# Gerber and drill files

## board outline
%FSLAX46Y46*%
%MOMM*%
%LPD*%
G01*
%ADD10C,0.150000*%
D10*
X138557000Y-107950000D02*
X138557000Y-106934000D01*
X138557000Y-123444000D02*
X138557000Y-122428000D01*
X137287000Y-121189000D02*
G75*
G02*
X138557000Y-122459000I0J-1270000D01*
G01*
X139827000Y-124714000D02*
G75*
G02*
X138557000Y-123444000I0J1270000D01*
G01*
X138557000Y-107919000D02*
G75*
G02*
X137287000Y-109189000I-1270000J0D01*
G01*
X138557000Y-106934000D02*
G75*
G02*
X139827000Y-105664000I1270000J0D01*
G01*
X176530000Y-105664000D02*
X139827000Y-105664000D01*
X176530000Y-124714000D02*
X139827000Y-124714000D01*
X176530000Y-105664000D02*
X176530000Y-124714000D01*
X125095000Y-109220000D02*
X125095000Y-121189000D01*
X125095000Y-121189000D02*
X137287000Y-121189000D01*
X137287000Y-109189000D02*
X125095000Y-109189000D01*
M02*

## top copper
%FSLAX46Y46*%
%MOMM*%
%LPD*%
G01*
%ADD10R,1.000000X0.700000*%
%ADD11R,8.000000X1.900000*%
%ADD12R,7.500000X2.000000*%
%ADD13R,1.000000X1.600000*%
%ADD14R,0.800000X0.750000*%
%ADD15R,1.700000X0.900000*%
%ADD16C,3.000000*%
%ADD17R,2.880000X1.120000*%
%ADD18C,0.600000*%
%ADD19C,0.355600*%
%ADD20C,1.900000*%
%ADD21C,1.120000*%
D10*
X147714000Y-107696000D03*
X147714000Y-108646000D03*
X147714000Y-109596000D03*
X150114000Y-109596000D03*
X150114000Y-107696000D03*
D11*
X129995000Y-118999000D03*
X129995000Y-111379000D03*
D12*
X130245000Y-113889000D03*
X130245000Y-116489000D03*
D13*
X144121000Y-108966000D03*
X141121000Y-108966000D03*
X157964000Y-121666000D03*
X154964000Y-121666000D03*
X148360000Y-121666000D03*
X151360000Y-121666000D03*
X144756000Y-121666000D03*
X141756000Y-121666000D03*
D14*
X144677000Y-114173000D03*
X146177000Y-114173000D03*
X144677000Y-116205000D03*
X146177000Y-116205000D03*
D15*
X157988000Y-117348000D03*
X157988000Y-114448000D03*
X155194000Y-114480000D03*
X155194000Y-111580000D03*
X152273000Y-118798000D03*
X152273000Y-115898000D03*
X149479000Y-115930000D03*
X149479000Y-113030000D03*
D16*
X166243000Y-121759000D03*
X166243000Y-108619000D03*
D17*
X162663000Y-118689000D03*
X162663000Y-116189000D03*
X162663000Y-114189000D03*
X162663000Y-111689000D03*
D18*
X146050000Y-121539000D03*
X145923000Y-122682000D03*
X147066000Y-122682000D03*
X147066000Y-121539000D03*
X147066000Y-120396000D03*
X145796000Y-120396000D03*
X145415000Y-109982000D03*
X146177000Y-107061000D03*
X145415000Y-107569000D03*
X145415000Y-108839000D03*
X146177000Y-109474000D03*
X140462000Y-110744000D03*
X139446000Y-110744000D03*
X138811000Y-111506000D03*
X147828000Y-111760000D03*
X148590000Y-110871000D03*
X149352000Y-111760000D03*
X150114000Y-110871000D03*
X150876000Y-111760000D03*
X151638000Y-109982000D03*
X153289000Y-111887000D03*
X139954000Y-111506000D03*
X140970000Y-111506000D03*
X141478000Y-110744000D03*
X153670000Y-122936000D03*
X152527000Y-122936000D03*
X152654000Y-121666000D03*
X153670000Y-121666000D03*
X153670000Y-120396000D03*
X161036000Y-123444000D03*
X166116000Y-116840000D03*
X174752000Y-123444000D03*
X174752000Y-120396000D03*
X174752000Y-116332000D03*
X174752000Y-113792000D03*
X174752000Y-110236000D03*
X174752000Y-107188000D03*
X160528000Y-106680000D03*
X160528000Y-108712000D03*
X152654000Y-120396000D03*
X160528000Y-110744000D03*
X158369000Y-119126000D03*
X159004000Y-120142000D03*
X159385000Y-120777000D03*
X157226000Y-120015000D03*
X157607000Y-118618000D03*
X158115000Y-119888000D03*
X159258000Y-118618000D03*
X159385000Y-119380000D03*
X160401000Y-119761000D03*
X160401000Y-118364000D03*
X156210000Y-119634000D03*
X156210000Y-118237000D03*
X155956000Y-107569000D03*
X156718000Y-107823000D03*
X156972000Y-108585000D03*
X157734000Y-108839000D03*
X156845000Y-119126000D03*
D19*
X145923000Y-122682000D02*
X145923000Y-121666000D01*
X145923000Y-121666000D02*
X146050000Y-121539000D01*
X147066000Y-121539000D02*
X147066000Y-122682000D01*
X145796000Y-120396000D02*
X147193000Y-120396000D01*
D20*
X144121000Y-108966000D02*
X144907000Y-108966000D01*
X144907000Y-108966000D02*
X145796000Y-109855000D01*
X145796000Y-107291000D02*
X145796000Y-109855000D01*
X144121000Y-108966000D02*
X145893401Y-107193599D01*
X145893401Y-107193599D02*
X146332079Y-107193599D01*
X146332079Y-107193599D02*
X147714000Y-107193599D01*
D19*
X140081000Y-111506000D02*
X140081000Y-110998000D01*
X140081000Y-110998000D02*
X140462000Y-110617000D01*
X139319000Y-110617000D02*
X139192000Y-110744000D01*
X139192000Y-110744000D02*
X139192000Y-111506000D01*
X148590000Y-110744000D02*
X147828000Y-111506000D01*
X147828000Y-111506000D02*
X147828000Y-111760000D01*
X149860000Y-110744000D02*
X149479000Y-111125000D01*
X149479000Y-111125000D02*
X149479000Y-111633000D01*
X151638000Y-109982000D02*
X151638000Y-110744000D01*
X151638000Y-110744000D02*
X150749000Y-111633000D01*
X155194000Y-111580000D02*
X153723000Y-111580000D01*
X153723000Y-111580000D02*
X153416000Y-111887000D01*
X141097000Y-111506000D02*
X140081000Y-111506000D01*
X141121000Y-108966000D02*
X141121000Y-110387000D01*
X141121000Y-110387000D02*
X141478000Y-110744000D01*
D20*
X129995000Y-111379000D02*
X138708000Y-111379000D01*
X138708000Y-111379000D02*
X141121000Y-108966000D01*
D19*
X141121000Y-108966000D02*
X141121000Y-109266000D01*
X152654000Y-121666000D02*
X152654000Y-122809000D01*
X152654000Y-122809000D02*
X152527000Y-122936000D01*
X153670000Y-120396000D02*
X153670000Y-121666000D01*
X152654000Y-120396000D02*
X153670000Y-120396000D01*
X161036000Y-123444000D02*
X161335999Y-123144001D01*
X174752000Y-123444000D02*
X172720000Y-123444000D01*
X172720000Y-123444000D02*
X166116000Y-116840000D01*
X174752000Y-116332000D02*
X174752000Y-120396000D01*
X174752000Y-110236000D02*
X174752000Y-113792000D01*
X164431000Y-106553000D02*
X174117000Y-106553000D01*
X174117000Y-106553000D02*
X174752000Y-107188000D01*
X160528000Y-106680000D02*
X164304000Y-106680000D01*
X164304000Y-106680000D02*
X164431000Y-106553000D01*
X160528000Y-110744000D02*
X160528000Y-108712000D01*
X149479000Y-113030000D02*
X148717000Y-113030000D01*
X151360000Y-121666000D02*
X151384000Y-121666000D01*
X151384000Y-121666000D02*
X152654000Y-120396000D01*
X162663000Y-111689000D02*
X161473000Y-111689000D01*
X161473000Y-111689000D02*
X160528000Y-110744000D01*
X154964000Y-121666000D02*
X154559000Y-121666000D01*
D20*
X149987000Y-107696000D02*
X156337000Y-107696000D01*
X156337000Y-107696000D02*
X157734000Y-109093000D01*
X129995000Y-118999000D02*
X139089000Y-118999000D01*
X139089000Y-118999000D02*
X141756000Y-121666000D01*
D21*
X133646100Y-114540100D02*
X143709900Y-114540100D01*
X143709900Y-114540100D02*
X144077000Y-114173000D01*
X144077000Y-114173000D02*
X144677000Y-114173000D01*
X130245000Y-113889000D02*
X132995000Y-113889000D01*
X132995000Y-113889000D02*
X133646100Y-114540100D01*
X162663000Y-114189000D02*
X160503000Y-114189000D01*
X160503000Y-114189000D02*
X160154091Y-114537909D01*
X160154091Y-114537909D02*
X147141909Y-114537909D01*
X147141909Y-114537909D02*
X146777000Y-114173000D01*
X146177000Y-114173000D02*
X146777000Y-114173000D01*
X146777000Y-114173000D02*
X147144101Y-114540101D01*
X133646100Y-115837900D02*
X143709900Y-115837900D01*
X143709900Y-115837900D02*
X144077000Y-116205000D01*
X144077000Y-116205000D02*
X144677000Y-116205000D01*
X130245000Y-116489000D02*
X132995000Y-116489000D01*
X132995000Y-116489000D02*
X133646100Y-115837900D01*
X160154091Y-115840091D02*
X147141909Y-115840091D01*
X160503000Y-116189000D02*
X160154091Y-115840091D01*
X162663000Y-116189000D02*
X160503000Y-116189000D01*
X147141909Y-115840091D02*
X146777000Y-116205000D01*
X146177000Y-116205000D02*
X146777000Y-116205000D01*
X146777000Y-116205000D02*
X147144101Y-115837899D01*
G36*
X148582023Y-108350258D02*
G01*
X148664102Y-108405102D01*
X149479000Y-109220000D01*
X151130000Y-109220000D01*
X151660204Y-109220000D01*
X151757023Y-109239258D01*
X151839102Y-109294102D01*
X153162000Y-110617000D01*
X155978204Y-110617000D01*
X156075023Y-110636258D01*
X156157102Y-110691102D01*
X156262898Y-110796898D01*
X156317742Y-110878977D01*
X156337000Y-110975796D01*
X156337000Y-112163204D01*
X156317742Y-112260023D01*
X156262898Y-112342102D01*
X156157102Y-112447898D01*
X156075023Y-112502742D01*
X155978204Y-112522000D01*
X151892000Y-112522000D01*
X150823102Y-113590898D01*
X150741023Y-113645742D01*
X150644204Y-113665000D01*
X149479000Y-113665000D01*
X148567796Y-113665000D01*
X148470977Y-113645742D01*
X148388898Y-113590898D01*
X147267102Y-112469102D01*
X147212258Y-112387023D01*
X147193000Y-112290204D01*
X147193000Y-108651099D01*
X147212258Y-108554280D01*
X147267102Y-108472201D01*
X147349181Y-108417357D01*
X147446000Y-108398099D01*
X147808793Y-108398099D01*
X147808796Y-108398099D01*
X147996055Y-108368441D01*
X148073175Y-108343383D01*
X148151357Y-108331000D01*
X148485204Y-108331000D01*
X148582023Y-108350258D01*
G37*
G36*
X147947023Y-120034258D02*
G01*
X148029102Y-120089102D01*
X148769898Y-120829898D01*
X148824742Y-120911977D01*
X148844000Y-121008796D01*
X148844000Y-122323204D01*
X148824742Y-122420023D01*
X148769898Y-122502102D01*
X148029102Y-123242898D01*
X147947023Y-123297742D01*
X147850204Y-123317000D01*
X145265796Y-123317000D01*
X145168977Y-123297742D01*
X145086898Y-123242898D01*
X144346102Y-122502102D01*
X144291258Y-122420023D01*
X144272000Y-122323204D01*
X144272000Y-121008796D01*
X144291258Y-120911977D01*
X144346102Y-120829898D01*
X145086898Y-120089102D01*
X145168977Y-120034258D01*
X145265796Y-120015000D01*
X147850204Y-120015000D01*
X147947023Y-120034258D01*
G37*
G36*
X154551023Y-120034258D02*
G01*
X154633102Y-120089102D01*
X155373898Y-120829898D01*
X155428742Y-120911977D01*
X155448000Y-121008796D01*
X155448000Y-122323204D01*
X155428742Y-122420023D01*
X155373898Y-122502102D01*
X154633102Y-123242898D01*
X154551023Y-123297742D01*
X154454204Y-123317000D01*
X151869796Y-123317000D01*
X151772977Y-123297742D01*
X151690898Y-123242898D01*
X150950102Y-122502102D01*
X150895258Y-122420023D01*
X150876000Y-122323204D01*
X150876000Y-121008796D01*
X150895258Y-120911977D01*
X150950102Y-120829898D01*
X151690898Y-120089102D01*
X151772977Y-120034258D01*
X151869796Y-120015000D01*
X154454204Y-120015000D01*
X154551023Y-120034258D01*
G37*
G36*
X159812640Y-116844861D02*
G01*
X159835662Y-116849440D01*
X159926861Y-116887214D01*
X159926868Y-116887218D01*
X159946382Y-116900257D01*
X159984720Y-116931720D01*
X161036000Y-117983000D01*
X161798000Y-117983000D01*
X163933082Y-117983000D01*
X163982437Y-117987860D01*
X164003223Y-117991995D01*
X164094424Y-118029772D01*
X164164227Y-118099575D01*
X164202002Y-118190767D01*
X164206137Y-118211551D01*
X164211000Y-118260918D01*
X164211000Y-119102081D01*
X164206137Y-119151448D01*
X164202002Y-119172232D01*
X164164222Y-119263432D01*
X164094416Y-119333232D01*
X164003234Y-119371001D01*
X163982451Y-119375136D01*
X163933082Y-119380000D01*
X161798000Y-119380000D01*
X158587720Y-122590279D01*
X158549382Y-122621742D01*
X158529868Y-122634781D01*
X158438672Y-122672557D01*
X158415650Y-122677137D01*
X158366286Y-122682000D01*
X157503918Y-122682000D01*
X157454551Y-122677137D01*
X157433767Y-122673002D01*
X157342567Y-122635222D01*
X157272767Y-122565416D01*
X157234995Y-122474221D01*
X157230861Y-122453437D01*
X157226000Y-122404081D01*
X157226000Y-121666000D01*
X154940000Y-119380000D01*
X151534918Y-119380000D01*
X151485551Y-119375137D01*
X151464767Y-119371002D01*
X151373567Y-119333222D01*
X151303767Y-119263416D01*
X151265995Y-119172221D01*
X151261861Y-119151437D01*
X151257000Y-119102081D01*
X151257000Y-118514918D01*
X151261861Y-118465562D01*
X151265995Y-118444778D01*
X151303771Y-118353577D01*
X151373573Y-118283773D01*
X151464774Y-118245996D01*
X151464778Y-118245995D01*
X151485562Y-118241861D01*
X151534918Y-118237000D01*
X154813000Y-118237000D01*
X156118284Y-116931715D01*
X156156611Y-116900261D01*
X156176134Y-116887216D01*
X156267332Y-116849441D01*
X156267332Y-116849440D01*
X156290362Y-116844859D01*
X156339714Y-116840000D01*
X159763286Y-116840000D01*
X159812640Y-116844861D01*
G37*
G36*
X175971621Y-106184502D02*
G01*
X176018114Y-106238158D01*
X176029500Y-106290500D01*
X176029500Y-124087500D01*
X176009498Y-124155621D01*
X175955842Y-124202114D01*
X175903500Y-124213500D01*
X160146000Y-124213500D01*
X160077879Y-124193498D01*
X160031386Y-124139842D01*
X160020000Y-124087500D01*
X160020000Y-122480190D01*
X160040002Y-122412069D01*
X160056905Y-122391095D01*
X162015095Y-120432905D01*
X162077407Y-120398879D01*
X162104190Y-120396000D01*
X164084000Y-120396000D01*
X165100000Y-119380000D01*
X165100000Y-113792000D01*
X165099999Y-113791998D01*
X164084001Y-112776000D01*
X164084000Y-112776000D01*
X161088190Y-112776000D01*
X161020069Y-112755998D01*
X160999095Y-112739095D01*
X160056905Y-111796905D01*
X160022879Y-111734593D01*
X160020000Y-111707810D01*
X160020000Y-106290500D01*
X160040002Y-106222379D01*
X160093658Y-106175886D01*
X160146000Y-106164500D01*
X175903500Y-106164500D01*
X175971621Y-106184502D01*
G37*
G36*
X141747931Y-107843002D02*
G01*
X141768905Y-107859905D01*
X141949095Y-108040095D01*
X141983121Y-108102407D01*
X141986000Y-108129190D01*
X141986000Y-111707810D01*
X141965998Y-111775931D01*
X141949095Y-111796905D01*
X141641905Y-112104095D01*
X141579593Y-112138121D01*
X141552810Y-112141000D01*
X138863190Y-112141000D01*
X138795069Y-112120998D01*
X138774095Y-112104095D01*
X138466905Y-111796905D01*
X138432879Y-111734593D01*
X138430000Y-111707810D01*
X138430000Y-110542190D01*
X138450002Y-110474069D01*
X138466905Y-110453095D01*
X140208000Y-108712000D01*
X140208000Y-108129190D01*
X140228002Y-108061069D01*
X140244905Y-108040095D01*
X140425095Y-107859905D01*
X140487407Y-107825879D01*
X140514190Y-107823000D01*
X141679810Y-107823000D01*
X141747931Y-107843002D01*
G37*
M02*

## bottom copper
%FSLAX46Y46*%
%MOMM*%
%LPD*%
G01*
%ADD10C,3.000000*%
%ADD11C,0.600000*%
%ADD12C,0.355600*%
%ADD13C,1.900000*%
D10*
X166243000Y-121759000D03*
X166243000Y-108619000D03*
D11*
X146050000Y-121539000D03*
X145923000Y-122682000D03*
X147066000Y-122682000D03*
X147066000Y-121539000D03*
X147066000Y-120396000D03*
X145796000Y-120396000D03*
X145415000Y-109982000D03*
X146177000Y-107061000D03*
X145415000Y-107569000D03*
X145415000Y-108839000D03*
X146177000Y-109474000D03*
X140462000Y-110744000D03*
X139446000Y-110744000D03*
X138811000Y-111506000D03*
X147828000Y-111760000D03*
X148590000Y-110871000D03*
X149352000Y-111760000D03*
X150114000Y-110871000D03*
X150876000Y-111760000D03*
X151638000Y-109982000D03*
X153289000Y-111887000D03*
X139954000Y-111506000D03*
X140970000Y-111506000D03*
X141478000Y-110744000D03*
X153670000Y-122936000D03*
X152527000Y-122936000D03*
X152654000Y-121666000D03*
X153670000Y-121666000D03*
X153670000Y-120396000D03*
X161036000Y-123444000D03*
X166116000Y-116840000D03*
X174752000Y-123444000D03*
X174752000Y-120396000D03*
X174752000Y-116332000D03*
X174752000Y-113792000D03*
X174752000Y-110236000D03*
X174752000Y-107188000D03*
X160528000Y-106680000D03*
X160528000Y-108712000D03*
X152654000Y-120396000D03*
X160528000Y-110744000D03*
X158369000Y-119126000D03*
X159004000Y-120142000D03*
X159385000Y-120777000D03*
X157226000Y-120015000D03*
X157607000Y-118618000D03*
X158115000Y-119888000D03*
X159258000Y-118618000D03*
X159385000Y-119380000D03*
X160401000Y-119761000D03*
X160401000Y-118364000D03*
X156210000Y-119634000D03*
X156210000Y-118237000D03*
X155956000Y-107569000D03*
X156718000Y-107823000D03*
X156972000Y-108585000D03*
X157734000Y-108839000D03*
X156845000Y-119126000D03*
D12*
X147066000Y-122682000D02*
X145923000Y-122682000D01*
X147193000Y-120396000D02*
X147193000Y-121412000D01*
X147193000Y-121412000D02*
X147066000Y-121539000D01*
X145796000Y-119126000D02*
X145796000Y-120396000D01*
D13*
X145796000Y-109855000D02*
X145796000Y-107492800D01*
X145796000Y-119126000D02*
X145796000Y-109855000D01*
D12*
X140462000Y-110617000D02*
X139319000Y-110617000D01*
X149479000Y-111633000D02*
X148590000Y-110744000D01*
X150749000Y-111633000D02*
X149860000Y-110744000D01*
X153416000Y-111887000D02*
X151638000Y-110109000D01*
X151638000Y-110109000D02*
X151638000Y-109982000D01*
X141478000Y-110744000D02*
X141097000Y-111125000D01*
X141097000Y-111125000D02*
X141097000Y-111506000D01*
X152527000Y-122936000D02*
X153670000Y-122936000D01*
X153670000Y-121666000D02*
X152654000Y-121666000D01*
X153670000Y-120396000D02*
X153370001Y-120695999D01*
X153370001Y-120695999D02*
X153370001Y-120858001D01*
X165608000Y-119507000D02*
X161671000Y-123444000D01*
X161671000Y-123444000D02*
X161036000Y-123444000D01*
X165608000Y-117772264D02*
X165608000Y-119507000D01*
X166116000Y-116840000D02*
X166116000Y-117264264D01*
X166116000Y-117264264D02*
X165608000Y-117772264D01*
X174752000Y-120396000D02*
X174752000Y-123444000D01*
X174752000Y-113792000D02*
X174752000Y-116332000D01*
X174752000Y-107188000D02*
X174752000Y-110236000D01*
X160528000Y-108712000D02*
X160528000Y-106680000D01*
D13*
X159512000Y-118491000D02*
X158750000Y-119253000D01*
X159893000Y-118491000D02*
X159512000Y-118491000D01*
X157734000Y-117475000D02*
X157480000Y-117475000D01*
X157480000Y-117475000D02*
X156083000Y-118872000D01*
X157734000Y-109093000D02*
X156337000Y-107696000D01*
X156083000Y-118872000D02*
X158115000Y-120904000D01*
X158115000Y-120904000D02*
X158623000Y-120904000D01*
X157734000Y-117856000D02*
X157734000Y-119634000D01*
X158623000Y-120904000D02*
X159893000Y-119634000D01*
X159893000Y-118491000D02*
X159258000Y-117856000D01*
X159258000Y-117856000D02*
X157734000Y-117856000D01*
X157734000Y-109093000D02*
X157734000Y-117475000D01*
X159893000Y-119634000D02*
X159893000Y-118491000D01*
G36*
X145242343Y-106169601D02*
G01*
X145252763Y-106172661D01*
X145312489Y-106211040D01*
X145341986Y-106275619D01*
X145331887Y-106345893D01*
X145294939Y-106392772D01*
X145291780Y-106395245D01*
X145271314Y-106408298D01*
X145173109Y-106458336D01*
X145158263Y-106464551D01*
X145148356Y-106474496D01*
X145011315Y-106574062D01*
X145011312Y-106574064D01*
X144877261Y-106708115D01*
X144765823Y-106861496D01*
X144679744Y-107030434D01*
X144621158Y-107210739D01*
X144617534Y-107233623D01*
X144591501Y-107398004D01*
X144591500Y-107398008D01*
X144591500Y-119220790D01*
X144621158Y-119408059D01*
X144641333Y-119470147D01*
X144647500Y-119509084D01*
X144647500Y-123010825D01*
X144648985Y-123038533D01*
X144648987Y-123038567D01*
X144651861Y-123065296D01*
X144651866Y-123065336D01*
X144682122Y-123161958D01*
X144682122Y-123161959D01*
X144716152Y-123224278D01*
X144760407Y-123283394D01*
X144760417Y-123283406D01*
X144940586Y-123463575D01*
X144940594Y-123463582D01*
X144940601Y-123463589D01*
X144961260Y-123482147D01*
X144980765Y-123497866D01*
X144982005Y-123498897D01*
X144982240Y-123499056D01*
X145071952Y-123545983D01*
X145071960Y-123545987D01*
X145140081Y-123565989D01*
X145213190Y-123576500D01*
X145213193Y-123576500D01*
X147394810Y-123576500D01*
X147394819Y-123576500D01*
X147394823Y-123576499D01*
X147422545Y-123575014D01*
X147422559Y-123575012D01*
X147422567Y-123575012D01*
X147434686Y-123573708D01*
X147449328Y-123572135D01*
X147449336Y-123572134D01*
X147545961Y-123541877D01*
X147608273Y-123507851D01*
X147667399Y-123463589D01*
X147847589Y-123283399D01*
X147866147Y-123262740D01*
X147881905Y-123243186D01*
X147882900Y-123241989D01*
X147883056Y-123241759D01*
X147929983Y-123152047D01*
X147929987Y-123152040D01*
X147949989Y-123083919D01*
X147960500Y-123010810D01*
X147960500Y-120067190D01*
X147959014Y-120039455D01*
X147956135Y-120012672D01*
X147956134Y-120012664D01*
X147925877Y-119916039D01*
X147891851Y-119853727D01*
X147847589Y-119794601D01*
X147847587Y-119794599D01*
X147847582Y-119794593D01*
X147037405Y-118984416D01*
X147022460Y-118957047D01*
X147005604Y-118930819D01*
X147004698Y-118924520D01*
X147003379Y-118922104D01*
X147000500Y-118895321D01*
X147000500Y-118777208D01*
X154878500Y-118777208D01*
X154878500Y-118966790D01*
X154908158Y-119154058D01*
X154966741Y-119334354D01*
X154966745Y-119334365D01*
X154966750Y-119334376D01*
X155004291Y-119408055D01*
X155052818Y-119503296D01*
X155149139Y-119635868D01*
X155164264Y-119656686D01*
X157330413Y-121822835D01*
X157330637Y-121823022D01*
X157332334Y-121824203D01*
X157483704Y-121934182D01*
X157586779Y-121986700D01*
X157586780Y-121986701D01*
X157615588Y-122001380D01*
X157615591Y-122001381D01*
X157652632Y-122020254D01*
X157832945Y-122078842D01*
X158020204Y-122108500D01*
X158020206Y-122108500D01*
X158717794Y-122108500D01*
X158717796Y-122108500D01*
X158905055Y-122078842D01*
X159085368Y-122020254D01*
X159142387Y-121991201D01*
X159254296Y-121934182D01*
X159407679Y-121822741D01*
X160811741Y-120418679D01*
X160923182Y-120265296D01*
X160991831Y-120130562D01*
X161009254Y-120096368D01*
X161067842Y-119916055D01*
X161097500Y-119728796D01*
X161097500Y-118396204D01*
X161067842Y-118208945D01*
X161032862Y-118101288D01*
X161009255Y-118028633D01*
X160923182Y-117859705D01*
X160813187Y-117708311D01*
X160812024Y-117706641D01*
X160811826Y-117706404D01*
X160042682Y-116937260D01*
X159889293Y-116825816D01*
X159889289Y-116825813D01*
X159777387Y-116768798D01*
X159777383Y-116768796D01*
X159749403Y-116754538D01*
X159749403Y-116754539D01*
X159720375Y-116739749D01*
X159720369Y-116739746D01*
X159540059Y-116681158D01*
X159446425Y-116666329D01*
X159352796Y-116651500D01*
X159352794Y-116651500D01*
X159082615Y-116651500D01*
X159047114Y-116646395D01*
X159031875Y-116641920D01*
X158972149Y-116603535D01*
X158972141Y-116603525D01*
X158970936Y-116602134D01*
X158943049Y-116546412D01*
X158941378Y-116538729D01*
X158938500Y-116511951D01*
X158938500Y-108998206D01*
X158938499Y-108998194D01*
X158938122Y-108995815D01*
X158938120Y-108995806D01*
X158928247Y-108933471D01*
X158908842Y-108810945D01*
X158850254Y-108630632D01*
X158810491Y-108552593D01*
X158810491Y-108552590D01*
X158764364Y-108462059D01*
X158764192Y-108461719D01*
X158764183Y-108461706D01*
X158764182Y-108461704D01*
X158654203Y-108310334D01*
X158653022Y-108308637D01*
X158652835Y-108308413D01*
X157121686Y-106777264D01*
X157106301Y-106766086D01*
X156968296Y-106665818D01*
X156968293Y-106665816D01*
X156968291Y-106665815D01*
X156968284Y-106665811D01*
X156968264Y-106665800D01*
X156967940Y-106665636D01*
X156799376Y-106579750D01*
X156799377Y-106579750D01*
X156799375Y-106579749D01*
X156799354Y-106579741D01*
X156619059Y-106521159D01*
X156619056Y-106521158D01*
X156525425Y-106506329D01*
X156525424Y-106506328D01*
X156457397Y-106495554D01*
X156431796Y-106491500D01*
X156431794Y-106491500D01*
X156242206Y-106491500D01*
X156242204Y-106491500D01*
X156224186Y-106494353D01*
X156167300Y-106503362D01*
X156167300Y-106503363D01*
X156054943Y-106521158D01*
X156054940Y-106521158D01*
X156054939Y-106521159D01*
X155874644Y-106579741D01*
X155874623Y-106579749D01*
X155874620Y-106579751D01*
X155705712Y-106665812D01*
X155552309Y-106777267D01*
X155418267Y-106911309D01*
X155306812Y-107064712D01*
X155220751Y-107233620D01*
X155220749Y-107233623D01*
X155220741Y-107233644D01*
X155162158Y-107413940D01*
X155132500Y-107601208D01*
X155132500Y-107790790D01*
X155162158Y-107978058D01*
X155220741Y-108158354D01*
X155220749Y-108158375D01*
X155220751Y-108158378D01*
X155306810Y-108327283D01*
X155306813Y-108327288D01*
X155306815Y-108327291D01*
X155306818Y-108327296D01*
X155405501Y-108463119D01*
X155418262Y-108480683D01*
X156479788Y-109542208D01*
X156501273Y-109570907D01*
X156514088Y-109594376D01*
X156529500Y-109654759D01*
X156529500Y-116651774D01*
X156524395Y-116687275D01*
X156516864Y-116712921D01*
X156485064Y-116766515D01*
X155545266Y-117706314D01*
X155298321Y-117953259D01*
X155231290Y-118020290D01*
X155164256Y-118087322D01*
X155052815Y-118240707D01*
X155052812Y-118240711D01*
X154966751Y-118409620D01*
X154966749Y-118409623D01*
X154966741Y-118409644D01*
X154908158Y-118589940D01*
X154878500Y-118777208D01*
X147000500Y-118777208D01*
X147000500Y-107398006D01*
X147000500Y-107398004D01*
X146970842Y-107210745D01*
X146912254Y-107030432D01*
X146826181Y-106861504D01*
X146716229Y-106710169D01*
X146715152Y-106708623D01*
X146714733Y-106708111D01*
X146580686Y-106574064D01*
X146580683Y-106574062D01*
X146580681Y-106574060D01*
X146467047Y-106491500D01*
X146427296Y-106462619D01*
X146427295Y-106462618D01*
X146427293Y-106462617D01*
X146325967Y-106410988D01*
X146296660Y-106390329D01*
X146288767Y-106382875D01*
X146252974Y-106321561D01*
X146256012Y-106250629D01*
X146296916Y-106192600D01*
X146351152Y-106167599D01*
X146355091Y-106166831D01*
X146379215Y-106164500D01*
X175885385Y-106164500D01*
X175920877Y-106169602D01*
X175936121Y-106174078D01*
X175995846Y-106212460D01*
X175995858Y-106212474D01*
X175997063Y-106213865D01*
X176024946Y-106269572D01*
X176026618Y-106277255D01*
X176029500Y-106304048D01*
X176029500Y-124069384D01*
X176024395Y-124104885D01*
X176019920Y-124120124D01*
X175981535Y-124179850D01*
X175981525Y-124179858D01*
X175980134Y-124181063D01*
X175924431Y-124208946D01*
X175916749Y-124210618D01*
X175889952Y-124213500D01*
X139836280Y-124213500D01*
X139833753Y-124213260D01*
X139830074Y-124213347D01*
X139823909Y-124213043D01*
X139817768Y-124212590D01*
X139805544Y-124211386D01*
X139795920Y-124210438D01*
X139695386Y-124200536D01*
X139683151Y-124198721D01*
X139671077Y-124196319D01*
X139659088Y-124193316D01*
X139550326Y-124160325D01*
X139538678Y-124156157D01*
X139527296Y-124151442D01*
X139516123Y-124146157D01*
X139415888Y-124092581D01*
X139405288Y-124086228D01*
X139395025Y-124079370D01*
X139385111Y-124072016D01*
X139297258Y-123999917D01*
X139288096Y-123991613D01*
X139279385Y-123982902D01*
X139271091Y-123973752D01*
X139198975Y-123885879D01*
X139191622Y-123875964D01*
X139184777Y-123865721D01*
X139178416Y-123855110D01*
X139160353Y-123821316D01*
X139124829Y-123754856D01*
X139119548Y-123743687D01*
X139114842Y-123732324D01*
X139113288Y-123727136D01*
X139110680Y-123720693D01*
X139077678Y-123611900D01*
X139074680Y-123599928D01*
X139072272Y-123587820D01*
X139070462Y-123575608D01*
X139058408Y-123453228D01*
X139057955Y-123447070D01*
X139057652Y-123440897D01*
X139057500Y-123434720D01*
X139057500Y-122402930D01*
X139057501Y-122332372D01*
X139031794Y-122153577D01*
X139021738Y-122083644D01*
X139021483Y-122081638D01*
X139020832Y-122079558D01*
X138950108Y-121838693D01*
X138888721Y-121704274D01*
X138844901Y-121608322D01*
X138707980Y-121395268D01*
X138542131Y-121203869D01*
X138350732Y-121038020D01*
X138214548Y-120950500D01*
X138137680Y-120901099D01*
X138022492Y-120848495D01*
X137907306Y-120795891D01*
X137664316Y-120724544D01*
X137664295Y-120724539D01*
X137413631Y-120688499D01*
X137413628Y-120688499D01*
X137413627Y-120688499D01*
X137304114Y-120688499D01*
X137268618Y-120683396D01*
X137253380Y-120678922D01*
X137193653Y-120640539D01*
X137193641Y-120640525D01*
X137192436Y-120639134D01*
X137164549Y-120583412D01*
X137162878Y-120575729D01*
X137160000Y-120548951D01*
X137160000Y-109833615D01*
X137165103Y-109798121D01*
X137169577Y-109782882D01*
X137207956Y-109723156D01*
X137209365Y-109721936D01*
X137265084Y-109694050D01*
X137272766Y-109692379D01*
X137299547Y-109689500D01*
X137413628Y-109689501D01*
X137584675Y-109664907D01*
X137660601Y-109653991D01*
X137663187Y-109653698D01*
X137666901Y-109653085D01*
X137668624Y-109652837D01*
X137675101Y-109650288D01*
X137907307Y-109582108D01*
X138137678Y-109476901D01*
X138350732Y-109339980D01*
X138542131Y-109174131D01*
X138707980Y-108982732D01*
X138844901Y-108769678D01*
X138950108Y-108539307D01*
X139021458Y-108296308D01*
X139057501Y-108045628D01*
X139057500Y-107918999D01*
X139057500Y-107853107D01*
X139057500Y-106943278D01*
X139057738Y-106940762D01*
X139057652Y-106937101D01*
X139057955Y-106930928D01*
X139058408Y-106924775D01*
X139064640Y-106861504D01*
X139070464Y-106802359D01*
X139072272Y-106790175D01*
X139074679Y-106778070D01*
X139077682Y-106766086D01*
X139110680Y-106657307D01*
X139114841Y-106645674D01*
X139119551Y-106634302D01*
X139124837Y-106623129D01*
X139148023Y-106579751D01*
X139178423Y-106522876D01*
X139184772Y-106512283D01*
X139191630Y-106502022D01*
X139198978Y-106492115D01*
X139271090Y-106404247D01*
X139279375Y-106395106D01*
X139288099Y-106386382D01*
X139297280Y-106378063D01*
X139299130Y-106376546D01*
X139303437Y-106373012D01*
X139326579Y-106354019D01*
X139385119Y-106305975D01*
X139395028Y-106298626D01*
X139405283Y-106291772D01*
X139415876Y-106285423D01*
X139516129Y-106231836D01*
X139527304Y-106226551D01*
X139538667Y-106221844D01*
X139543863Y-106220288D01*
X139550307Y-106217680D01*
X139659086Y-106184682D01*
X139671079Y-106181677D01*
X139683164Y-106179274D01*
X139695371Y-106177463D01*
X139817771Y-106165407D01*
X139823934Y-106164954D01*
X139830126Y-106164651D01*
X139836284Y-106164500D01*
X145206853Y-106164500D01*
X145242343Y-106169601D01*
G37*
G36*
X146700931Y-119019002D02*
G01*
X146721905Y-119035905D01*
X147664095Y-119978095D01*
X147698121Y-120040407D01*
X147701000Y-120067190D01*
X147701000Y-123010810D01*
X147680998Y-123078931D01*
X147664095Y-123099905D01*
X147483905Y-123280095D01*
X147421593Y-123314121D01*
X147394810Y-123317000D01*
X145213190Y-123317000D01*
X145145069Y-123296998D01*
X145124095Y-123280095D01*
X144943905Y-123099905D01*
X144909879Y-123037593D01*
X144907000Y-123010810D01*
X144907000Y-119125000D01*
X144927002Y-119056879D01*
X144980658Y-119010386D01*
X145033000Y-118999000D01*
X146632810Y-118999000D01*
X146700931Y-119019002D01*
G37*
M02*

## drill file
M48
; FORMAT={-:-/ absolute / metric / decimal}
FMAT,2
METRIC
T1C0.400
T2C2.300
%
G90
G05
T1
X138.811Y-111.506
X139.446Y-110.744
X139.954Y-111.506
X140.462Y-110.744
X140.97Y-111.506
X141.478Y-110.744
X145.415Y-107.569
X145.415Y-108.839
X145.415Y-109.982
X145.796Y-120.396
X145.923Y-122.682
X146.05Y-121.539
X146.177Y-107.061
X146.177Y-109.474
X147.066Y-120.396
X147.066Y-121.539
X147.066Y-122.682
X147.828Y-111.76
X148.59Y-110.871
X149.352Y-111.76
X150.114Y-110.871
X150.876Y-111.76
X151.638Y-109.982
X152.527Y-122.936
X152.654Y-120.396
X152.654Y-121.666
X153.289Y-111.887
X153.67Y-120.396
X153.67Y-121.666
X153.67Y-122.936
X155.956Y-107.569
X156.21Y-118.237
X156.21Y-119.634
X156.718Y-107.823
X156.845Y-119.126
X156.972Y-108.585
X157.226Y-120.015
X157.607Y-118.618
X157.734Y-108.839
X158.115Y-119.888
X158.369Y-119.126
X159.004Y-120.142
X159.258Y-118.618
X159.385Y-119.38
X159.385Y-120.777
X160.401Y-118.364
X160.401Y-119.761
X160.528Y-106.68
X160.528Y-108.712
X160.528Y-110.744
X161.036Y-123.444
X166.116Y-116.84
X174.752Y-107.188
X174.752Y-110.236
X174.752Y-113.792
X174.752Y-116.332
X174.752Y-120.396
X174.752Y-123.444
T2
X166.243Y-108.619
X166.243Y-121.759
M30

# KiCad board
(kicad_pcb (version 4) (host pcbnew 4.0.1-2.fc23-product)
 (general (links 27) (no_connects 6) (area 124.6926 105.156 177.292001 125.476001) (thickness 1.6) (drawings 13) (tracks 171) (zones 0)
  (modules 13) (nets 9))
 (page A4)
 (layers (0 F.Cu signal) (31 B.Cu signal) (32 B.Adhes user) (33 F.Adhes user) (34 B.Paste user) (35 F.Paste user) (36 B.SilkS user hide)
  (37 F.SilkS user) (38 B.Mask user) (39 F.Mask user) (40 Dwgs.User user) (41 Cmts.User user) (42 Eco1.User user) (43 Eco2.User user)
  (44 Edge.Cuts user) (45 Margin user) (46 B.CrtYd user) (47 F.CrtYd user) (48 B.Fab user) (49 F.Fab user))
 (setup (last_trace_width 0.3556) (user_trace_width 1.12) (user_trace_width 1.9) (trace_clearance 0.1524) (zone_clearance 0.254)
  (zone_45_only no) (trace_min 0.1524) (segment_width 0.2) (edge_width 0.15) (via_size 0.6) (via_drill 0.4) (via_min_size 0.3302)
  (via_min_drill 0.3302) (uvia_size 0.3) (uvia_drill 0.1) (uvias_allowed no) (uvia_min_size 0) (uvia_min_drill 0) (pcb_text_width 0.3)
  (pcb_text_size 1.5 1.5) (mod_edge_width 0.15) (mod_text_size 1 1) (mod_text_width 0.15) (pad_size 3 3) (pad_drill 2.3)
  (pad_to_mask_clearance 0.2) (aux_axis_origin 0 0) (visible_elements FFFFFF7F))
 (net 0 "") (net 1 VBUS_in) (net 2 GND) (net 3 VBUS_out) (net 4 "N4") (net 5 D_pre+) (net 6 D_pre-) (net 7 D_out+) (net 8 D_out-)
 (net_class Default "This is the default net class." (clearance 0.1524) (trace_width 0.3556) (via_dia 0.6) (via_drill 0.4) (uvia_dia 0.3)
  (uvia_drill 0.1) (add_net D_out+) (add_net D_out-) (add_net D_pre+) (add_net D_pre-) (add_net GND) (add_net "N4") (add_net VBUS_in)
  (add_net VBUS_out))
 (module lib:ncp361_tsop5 (layer F.Cu) (at 148.914 108.646 270)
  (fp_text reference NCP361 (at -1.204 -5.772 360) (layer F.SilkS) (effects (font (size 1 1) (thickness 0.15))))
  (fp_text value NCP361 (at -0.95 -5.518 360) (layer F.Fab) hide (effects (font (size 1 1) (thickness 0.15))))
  (pad 1 smd rect (at -0.95 1.2 270) (size 0.7 1) (layers F.Cu F.Paste F.Mask) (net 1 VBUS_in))
  (pad 2 smd rect (at 0 1.2 270) (size 0.7 1) (layers F.Cu F.Paste F.Mask) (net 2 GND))
  (pad 3 smd rect (at 0.95 1.2 270) (size 0.7 1) (layers F.Cu F.Paste F.Mask) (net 2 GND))
  (pad 4 smd rect (at 0.95 -1.2 270) (size 0.7 1) (layers F.Cu F.Paste F.Mask) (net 2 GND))
  (pad 5 smd rect (at -0.95 -1.2 270) (size 0.7 1) (layers F.Cu F.Paste F.Mask) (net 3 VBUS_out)))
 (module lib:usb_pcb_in (layer F.Cu) (at 125.095 115.189 270)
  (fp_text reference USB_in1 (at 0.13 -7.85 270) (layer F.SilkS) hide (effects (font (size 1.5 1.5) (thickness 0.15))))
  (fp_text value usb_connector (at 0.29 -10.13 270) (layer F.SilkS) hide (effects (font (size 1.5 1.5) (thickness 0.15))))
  (pad 1 connect rect (at 3.81 -4.9 270) (size 1.9 8) (layers F.Cu F.Mask) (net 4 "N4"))
  (pad 4 connect rect (at -3.81 -4.9 270) (size 1.9 8) (layers F.Cu F.Mask) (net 2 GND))
  (pad 3 connect rect (at -1.3 -5.15 270) (size 2 7.5) (layers F.Cu F.Mask) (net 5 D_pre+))
  (pad 2 connect rect (at 1.3 -5.15 270) (size 2 7.5) (layers F.Cu F.Mask) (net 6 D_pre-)))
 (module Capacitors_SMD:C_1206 (layer F.Cu) (at 142.621 108.966 180)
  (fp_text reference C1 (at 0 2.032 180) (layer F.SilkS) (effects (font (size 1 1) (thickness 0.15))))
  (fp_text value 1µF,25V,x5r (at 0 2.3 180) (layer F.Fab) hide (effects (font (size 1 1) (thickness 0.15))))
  (pad 1 smd rect (at -1.5 0 180) (size 1 1.6) (layers F.Cu F.Paste F.Mask) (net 1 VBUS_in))
  (pad 2 smd rect (at 1.5 0 180) (size 1 1.6) (layers F.Cu F.Paste F.Mask) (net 2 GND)))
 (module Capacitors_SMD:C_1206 (layer F.Cu) (at 156.464 121.666 180)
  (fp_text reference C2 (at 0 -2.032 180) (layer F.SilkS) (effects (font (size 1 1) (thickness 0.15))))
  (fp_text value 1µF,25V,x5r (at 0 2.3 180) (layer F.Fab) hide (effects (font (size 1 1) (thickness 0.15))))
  (pad 1 smd rect (at -1.5 0 180) (size 1 1.6) (layers F.Cu F.Paste F.Mask) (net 3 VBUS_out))
  (pad 2 smd rect (at 1.5 0 180) (size 1 1.6) (layers F.Cu F.Paste F.Mask) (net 2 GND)))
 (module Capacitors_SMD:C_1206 (layer F.Cu) (at 149.86 121.666)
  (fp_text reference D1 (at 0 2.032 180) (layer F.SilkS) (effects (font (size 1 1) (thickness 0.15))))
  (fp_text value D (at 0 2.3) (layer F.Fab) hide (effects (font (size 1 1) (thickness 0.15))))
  (pad 1 smd rect (at -1.5 0) (size 1 1.6) (layers F.Cu F.Paste F.Mask) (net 1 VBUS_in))
  (pad 2 smd rect (at 1.5 0) (size 1 1.6) (layers F.Cu F.Paste F.Mask) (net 2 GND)))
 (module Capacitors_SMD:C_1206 (layer F.Cu) (at 143.256 121.666 180)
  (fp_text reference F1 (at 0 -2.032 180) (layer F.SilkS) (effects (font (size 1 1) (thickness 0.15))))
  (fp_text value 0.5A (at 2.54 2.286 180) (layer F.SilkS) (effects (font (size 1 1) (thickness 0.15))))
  (pad 1 smd rect (at -1.5 0 180) (size 1 1.6) (layers F.Cu F.Paste F.Mask) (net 1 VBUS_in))
  (pad 2 smd rect (at 1.5 0 180) (size 1 1.6) (layers F.Cu F.Paste F.Mask) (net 4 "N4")))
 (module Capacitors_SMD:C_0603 (layer F.Cu) (at 145.427 114.173)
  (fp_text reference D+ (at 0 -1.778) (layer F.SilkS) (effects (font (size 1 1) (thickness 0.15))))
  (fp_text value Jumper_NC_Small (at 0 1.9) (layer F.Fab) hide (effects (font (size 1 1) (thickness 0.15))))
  (pad 1 smd rect (at -0.75 0) (size 0.8 0.75) (layers F.Cu F.Paste F.Mask) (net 5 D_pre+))
  (pad 2 smd rect (at 0.75 0) (size 0.8 0.75) (layers F.Cu F.Paste F.Mask) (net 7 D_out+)))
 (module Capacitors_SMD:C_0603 (layer F.Cu) (at 145.427 116.205)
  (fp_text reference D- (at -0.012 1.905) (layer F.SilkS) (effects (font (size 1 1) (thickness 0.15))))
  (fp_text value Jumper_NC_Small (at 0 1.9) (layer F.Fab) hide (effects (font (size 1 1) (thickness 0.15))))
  (pad 1 smd rect (at -0.75 0) (size 0.8 0.75) (layers F.Cu F.Paste F.Mask) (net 6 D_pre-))
  (pad 2 smd rect (at 0.75 0) (size 0.8 0.75) (layers F.Cu F.Paste F.Mask) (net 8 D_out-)))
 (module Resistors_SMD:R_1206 (layer F.Cu) (at 157.988 115.898 90)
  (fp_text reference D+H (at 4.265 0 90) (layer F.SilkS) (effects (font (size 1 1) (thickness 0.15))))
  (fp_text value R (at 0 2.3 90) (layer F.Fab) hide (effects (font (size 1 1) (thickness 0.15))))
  (pad 1 smd rect (at -1.45 0 90) (size 0.9 1.7) (layers F.Cu F.Paste F.Mask) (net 3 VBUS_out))
  (pad 2 smd rect (at 1.45 0 90) (size 0.9 1.7) (layers F.Cu F.Paste F.Mask) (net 7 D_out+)))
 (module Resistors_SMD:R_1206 (layer F.Cu) (at 155.194 113.03 90)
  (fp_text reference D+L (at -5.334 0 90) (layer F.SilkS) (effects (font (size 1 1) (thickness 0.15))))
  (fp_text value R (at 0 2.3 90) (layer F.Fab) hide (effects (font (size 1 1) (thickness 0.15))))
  (pad 1 smd rect (at -1.45 0 90) (size 0.9 1.7) (layers F.Cu F.Paste F.Mask) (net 7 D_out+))
  (pad 2 smd rect (at 1.45 0 90) (size 0.9 1.7) (layers F.Cu F.Paste F.Mask) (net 2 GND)))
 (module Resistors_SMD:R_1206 (layer F.Cu) (at 152.273 117.348 90)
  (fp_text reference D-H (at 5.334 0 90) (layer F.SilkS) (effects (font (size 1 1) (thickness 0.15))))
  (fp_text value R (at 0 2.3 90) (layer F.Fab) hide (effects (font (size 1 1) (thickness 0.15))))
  (pad 1 smd rect (at -1.45 0 90) (size 0.9 1.7) (layers F.Cu F.Paste F.Mask) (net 3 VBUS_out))
  (pad 2 smd rect (at 1.45 0 90) (size 0.9 1.7) (layers F.Cu F.Paste F.Mask) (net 8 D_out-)))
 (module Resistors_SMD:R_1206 (layer F.Cu) (at 149.479 114.48 90)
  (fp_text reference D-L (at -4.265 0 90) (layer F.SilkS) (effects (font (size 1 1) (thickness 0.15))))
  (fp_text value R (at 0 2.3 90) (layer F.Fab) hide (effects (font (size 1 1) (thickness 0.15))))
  (pad 1 smd rect (at -1.45 0 90) (size 0.9 1.7) (layers F.Cu F.Paste F.Mask) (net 8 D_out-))
  (pad 2 smd rect (at 1.45 0 90) (size 0.9 1.7) (layers F.Cu F.Paste F.Mask) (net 2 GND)))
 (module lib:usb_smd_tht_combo (layer F.Cu) (at 166.243 115.189 90)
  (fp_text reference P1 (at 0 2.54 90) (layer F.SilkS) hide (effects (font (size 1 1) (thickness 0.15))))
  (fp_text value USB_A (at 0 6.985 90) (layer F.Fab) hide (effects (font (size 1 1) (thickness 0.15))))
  (pad 5 thru_hole circle (at -6.57 0 90) (size 3 3) (drill 2.3) (layers *.Cu *.Mask F.SilkS) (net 2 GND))
  (pad 6 thru_hole circle (at 6.57 0 90) (size 3 3) (drill 2.3) (layers *.Cu *.Mask F.SilkS) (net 2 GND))
  (pad 1 smd rect (at -3.5 -3.58 90) (size 1.12 2.88) (layers F.Cu F.Paste F.Mask) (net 3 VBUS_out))
  (pad 2 smd rect (at -1 -3.58 90) (size 1.12 2.88) (layers F.Cu F.Paste F.Mask) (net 8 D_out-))
  (pad 3 smd rect (at 1 -3.58 90) (size 1.12 2.88) (layers F.Cu F.Paste F.Mask) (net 7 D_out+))
  (pad 4 smd rect (at 3.5 -3.58 90) (size 1.12 2.88) (layers F.Cu F.Paste F.Mask) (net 2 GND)))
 (gr_line (start 138.557 107.95) (end 138.557 106.934) (layer Edge.Cuts) (width 0.15))
 (gr_line (start 138.557 123.444) (end 138.557 122.428) (layer Edge.Cuts) (width 0.15))
 (gr_arc (start 137.287 122.459) (end 137.287 121.189) (angle 90) (layer Edge.Cuts) (width 0.15))
 (gr_arc (start 139.827 123.444) (end 139.827 124.714) (angle 90) (layer Edge.Cuts) (width 0.15))
 (gr_arc (start 137.287 107.919) (end 138.557 107.919) (angle 90) (layer Edge.Cuts) (width 0.15))
 (gr_arc (start 139.827 106.934) (end 138.557 106.934) (angle 90) (layer Edge.Cuts) (width 0.15))
 (gr_line (start 176.53 105.664) (end 139.827 105.664) (layer Edge.Cuts) (width 0.15))
 (gr_line (start 176.53 124.714) (end 139.827 124.714) (layer Edge.Cuts) (width 0.15))
 (gr_line (start 176.53 105.664) (end 176.53 124.714) (layer Edge.Cuts) (width 0.15))
 (gr_line (start 125.095 109.22) (end 125.095 121.189) (layer Edge.Cuts) (width 0.15))
 (gr_line (start 125.095 121.189) (end 137.287 121.189) (layer Edge.Cuts) (width 0.15))
 (gr_line (start 137.287 109.189) (end 125.095 109.189) (layer Edge.Cuts) (width 0.15))
 (segment (start 145.923 122.682) (end 145.923 121.666) (width 0.3556) (layer F.Cu) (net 1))
 (segment (start 145.923 121.666) (end 146.05 121.539) (width 0.3556) (layer F.Cu) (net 1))
 (via (at 146.05 121.539) (size 0.6) (drill 0.4) (layers F.Cu B.Cu) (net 1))
 (segment (start 147.066 122.682) (end 145.923 122.682) (width 0.3556) (layer B.Cu) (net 1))
 (via (at 145.923 122.682) (size 0.6) (drill 0.4) (layers F.Cu B.Cu) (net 1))
 (segment (start 147.066 121.539) (end 147.066 122.682) (width 0.3556) (layer F.Cu) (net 1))
 (via (at 147.066 122.682) (size 0.6) (drill 0.4) (layers F.Cu B.Cu) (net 1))
 (segment (start 147.193 120.396) (end 147.193 121.412) (width 0.3556) (layer B.Cu) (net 1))
 (segment (start 147.193 121.412) (end 147.066 121.539) (width 0.3556) (layer B.Cu) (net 1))
 (via (at 147.066 121.539) (size 0.6) (drill 0.4) (layers F.Cu B.Cu) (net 1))
 (segment (start 145.796 120.396) (end 147.193 120.396) (width 0.3556) (layer F.Cu) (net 1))
 (via (at 147.066 120.396) (size 0.6) (drill 0.4) (layers F.Cu B.Cu) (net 1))
 (segment (start 145.796 119.126) (end 145.796 120.396) (width 0.3556) (layer B.Cu) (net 1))
 (via (at 145.796 120.396) (size 0.6) (drill 0.4) (layers F.Cu B.Cu) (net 1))
 (segment (start 145.796 109.855) (end 145.796 107.4928) (width 1.9) (layer B.Cu) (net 1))
 (via (at 145.415 109.982) (size 0.6) (drill 0.4) (layers F.Cu B.Cu) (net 1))
 (via (at 146.177 107.061) (size 0.6) (drill 0.4) (layers F.Cu B.Cu) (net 1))
 (via (at 145.415 107.569) (size 0.6) (drill 0.4) (layers F.Cu B.Cu) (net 1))
 (via (at 145.415 108.839) (size 0.6) (drill 0.4) (layers F.Cu B.Cu) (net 1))
 (segment (start 144.121 108.966) (end 144.907 108.966) (width 1.9) (layer F.Cu) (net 1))
 (segment (start 144.907 108.966) (end 145.796 109.855) (width 1.9) (layer F.Cu) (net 1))
 (segment (start 145.796 107.291) (end 145.796 109.855) (width 1.9) (layer F.Cu) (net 1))
 (segment (start 144.121 108.966) (end 145.893401 107.193599) (width 1.9) (layer F.Cu) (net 1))
 (segment (start 145.893401 107.193599) (end 146.332079 107.193599) (width 1.9) (layer F.Cu) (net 1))
 (segment (start 146.332079 107.193599) (end 147.714 107.193599) (width 1.9) (layer F.Cu) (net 1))
 (segment (start 145.796 119.126) (end 145.796 109.855) (width 1.9) (layer B.Cu) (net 1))
 (via (at 146.177 109.474) (size 0.6) (drill 0.4) (layers F.Cu B.Cu) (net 1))
 (segment (start 140.081 111.506) (end 140.081 110.998) (width 0.3556) (layer F.Cu) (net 2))
 (segment (start 140.081 110.998) (end 140.462 110.617) (width 0.3556) (layer F.Cu) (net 2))
 (via (at 140.462 110.744) (size 0.6) (drill 0.4) (layers F.Cu B.Cu) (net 2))
 (segment (start 140.462 110.617) (end 139.319 110.617) (width 0.3556) (layer B.Cu) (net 2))
 (via (at 139.446 110.744) (size 0.6) (drill 0.4) (layers F.Cu B.Cu) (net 2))
 (segment (start 139.319 110.617) (end 139.192 110.744) (width 0.3556) (layer F.Cu) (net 2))
 (segment (start 139.192 110.744) (end 139.192 111.506) (width 0.3556) (layer F.Cu) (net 2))
 (via (at 138.811 111.506) (size 0.6) (drill 0.4) (layers F.Cu B.Cu) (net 2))
 (segment (start 148.59 110.744) (end 147.828 111.506) (width 0.3556) (layer F.Cu) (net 2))
 (segment (start 147.828 111.506) (end 147.828 111.76) (width 0.3556) (layer F.Cu) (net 2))
 (via (at 147.828 111.76) (size 0.6) (drill 0.4) (layers F.Cu B.Cu) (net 2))
 (segment (start 149.479 111.633) (end 148.59 110.744) (width 0.3556) (layer B.Cu) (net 2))
 (via (at 148.59 110.871) (size 0.6) (drill 0.4) (layers F.Cu B.Cu) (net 2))
 (segment (start 149.86 110.744) (end 149.479 111.125) (width 0.3556) (layer F.Cu) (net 2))
 (segment (start 149.479 111.125) (end 149.479 111.633) (width 0.3556) (layer F.Cu) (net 2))
 (via (at 149.352 111.76) (size 0.6) (drill 0.4) (layers F.Cu B.Cu) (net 2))
 (segment (start 150.749 111.633) (end 149.86 110.744) (width 0.3556) (layer B.Cu) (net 2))
 (via (at 150.114 110.871) (size 0.6) (drill 0.4) (layers F.Cu B.Cu) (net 2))
 (segment (start 151.638 109.982) (end 151.638 110.744) (width 0.3556) (layer F.Cu) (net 2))
 (segment (start 151.638 110.744) (end 150.749 111.633) (width 0.3556) (layer F.Cu) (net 2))
 (via (at 150.876 111.76) (size 0.6) (drill 0.4) (layers F.Cu B.Cu) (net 2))
 (segment (start 153.416 111.887) (end 151.638 110.109) (width 0.3556) (layer B.Cu) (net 2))
 (segment (start 151.638 110.109) (end 151.638 109.982) (width 0.3556) (layer B.Cu) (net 2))
 (via (at 151.638 109.982) (size 0.6) (drill 0.4) (layers F.Cu B.Cu) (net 2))
 (segment (start 155.194 111.58) (end 153.723 111.58) (width 0.3556) (layer F.Cu) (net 2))
 (segment (start 153.723 111.58) (end 153.416 111.887) (width 0.3556) (layer F.Cu) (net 2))
 (via (at 153.289 111.887) (size 0.6) (drill 0.4) (layers F.Cu B.Cu) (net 2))
 (segment (start 141.097 111.506) (end 140.081 111.506) (width 0.3556) (layer F.Cu) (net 2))
 (via (at 139.954 111.506) (size 0.6) (drill 0.4) (layers F.Cu B.Cu) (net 2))
 (segment (start 141.478 110.744) (end 141.097 111.125) (width 0.3556) (layer B.Cu) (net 2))
 (segment (start 141.097 111.125) (end 141.097 111.506) (width 0.3556) (layer B.Cu) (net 2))
 (via (at 140.97 111.506) (size 0.6) (drill 0.4) (layers F.Cu B.Cu) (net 2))
 (segment (start 141.121 108.966) (end 141.121 110.387) (width 0.3556) (layer F.Cu) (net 2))
 (segment (start 141.121 110.387) (end 141.478 110.744) (width 0.3556) (layer F.Cu) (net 2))
 (via (at 141.478 110.744) (size 0.6) (drill 0.4) (layers F.Cu B.Cu) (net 2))
 (segment (start 129.995 111.379) (end 138.708 111.379) (width 1.9) (layer F.Cu) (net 2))
 (segment (start 138.708 111.379) (end 141.121 108.966) (width 1.9) (layer F.Cu) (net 2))
 (segment (start 141.121 108.966) (end 141.121 109.266) (width 0.3556) (layer F.Cu) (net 2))
 (segment (start 152.527 122.936) (end 153.67 122.936) (width 0.3556) (layer B.Cu) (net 2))
 (via (at 153.67 122.936) (size 0.6) (drill 0.4) (layers F.Cu B.Cu) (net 2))
 (segment (start 152.654 121.666) (end 152.654 122.809) (width 0.3556) (layer F.Cu) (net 2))
 (segment (start 152.654 122.809) (end 152.527 122.936) (width 0.3556) (layer F.Cu) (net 2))
 (via (at 152.527 122.936) (size 0.6) (drill 0.4) (layers F.Cu B.Cu) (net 2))
 (segment (start 153.67 121.666) (end 152.654 121.666) (width 0.3556) (layer B.Cu) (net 2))
 (via (at 152.654 121.666) (size 0.6) (drill 0.4) (layers F.Cu B.Cu) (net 2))
 (segment (start 153.67 120.396) (end 153.67 121.666) (width 0.3556) (layer F.Cu) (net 2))
 (via (at 153.67 121.666) (size 0.6) (drill 0.4) (layers F.Cu B.Cu) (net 2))
 (segment (start 153.67 120.396) (end 153.370001 120.695999) (width 0.3556) (layer B.Cu) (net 2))
 (segment (start 153.370001 120.695999) (end 153.370001 120.858001) (width 0.3556) (layer B.Cu) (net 2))
 (segment (start 152.654 120.396) (end 153.67 120.396) (width 0.3556) (layer F.Cu) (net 2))
 (via (at 153.67 120.396) (size 0.6) (drill 0.4) (layers F.Cu B.Cu) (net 2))
 (segment (start 161.036 123.444) (end 161.335999 123.144001) (width 0.3556) (layer F.Cu) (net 2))
 (segment (start 165.608 119.507) (end 161.671 123.444) (width 0.3556) (layer B.Cu) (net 2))
 (segment (start 161.671 123.444) (end 161.036 123.444) (width 0.3556) (layer B.Cu) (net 2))
 (via (at 161.036 123.444) (size 0.6) (drill 0.4) (layers F.Cu B.Cu) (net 2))
 (segment (start 165.608 117.772264) (end 165.608 119.507) (width 0.3556) (layer B.Cu) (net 2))
 (segment (start 166.116 116.84) (end 166.116 117.264264) (width 0.3556) (layer B.Cu) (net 2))
 (segment (start 166.116 117.264264) (end 165.608 117.772264) (width 0.3556) (layer B.Cu) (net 2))
 (segment (start 174.752 123.444) (end 172.72 123.444) (width 0.3556) (layer F.Cu) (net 2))
 (segment (start 172.72 123.444) (end 166.116 116.84) (width 0.3556) (layer F.Cu) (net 2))
 (via (at 166.116 116.84) (size 0.6) (drill 0.4) (layers F.Cu B.Cu) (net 2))
 (segment (start 174.752 120.396) (end 174.752 123.444) (width 0.3556) (layer B.Cu) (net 2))
 (via (at 174.752 123.444) (size 0.6) (drill 0.4) (layers F.Cu B.Cu) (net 2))
 (segment (start 174.752 116.332) (end 174.752 120.396) (width 0.3556) (layer F.Cu) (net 2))
 (via (at 174.752 120.396) (size 0.6) (drill 0.4) (layers F.Cu B.Cu) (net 2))
 (segment (start 174.752 113.792) (end 174.752 116.332) (width 0.3556) (layer B.Cu) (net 2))
 (via (at 174.752 116.332) (size 0.6) (drill 0.4) (layers F.Cu B.Cu) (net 2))
 (segment (start 174.752 110.236) (end 174.752 113.792) (width 0.3556) (layer F.Cu) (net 2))
 (via (at 174.752 113.792) (size 0.6) (drill 0.4) (layers F.Cu B.Cu) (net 2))
 (segment (start 174.752 107.188) (end 174.752 110.236) (width 0.3556) (layer B.Cu) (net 2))
 (via (at 174.752 110.236) (size 0.6) (drill 0.4) (layers F.Cu B.Cu) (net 2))
 (segment (start 164.431 106.553) (end 174.117 106.553) (width 0.3556) (layer F.Cu) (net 2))
 (segment (start 174.117 106.553) (end 174.752 107.188) (width 0.3556) (layer F.Cu) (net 2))
 (via (at 174.752 107.188) (size 0.6) (drill 0.4) (layers F.Cu B.Cu) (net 2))
 (segment (start 160.528 106.68) (end 164.304 106.68) (width 0.3556) (layer F.Cu) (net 2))
 (segment (start 164.304 106.68) (end 164.431 106.553) (width 0.3556) (layer F.Cu) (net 2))
 (segment (start 160.528 108.712) (end 160.528 106.68) (width 0.3556) (layer B.Cu) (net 2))
 (via (at 160.528 106.68) (size 0.6) (drill 0.4) (layers F.Cu B.Cu) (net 2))
 (segment (start 160.528 110.744) (end 160.528 108.712) (width 0.3556) (layer F.Cu) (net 2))
 (via (at 160.528 108.712) (size 0.6) (drill 0.4) (layers F.Cu B.Cu) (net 2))
 (segment (start 149.479 113.03) (end 148.717 113.03) (width 0.3556) (layer F.Cu) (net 2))
 (segment (start 151.36 121.666) (end 151.384 121.666) (width 0.3556) (layer F.Cu) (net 2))
 (segment (start 151.384 121.666) (end 152.654 120.396) (width 0.3556) (layer F.Cu) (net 2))
 (via (at 152.654 120.396) (size 0.6) (drill 0.4) (layers F.Cu B.Cu) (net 2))
 (segment (start 162.663 111.689) (end 161.473 111.689) (width 0.3556) (layer F.Cu) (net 2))
 (segment (start 161.473 111.689) (end 160.528 110.744) (width 0.3556) (layer F.Cu) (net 2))
 (via (at 160.528 110.744) (size 0.6) (drill 0.4) (layers F.Cu B.Cu) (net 2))
 (segment (start 154.964 121.666) (end 154.559 121.666) (width 0.3556) (layer F.Cu) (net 2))
 (via (at 158.369 119.126) (size 0.6) (drill 0.4) (layers F.Cu B.Cu) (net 3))
 (via (at 159.004 120.142) (size 0.6) (drill 0.4) (layers F.Cu B.Cu) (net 3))
 (via (at 159.385 120.777) (size 0.6) (drill 0.4) (layers F.Cu B.Cu) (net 3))
 (via (at 157.226 120.015) (size 0.6) (drill 0.4) (layers F.Cu B.Cu) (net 3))
 (via (at 157.607 118.618) (size 0.6) (drill 0.4) (layers F.Cu B.Cu) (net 3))
 (via (at 158.115 119.888) (size 0.6) (drill 0.4) (layers F.Cu B.Cu) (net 3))
 (via (at 159.258 118.618) (size 0.6) (drill 0.4) (layers F.Cu B.Cu) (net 3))
 (via (at 159.385 119.38) (size 0.6) (drill 0.4) (layers F.Cu B.Cu) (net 3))
 (via (at 160.401 119.761) (size 0.6) (drill 0.4) (layers F.Cu B.Cu) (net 3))
 (via (at 160.401 118.364) (size 0.6) (drill 0.4) (layers F.Cu B.Cu) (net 3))
 (via (at 156.21 119.634) (size 0.6) (drill 0.4) (layers F.Cu B.Cu) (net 3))
 (via (at 156.21 118.237) (size 0.6) (drill 0.4) (layers F.Cu B.Cu) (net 3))
 (segment (start 159.512 118.491) (end 158.75 119.253) (width 1.9) (layer B.Cu) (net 3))
 (segment (start 159.893 118.491) (end 159.512 118.491) (width 1.9) (layer B.Cu) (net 3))
 (segment (start 157.734 117.475) (end 157.48 117.475) (width 1.9) (layer B.Cu) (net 3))
 (segment (start 157.48 117.475) (end 156.083 118.872) (width 1.9) (layer B.Cu) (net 3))
 (segment (start 157.734 109.093) (end 156.337 107.696) (width 1.9) (layer B.Cu) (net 3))
 (segment (start 156.083 118.872) (end 158.115 120.904) (width 1.9) (layer B.Cu) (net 3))
 (segment (start 158.115 120.904) (end 158.623 120.904) (width 1.9) (layer B.Cu) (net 3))
 (segment (start 157.734 117.856) (end 157.734 119.634) (width 1.9) (layer B.Cu) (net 3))
 (segment (start 158.623 120.904) (end 159.893 119.634) (width 1.9) (layer B.Cu) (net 3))
 (segment (start 159.893 118.491) (end 159.258 117.856) (width 1.9) (layer B.Cu) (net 3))
 (segment (start 159.258 117.856) (end 157.734 117.856) (width 1.9) (layer B.Cu) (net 3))
 (segment (start 157.734 109.093) (end 157.734 117.475) (width 1.9) (layer B.Cu) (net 3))
 (segment (start 159.893 119.634) (end 159.893 118.491) (width 1.9) (layer B.Cu) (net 3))
 (via (at 155.956 107.569) (size 0.6) (drill 0.4) (layers F.Cu B.Cu) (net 3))
 (via (at 156.718 107.823) (size 0.6) (drill 0.4) (layers F.Cu B.Cu) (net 3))
 (via (at 156.972 108.585) (size 0.6) (drill 0.4) (layers F.Cu B.Cu) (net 3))
 (via (at 157.734 108.839) (size 0.6) (drill 0.4) (layers F.Cu B.Cu) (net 3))
 (via (at 156.845 119.126) (size 0.6) (drill 0.4) (layers F.Cu B.Cu) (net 3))
 (segment (start 149.987 107.696) (end 156.337 107.696) (width 1.9) (layer F.Cu) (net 3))
 (segment (start 156.337 107.696) (end 157.734 109.093) (width 1.9) (layer F.Cu) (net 3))
 (segment (start 129.995 118.999) (end 139.089 118.999) (width 1.9) (layer F.Cu) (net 4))
 (segment (start 139.089 118.999) (end 141.756 121.666) (width 1.9) (layer F.Cu) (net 4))
 (segment (start 133.6461 114.5401) (end 143.7099 114.5401) (width 1.12) (layer F.Cu) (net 5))
 (segment (start 143.7099 114.5401) (end 144.077 114.173) (width 1.12) (layer F.Cu) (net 5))
 (segment (start 144.077 114.173) (end 144.677 114.173) (width 1.12) (layer F.Cu) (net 5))
 (segment (start 130.245 113.889) (end 132.995 113.889) (width 1.12) (layer F.Cu) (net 5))
 (segment (start 132.995 113.889) (end 133.6461 114.5401) (width 1.12) (layer F.Cu) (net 5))
 (segment (start 162.663 114.189) (end 160.503 114.189) (width 1.12) (layer F.Cu) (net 7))
 (segment (start 160.503 114.189) (end 160.154091 114.537909) (width 1.12) (layer F.Cu) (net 7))
 (segment (start 160.154091 114.537909) (end 147.141909 114.537909) (width 1.12) (layer F.Cu) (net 7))
 (segment (start 147.141909 114.537909) (end 146.777 114.173) (width 1.12) (layer F.Cu) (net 7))
 (segment (start 146.177 114.173) (end 146.777 114.173) (width 1.12) (layer F.Cu) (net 7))
 (segment (start 146.777 114.173) (end 147.144101 114.540101) (width 1.12) (layer F.Cu) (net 7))
 (segment (start 133.6461 115.8379) (end 143.7099 115.8379) (width 1.12) (layer F.Cu) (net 6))
 (segment (start 143.7099 115.8379) (end 144.077 116.205) (width 1.12) (layer F.Cu) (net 6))
 (segment (start 144.077 116.205) (end 144.677 116.205) (width 1.12) (layer F.Cu) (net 6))
 (segment (start 130.245 116.489) (end 132.995 116.489) (width 1.12) (layer F.Cu) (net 6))
 (segment (start 132.995 116.489) (end 133.6461 115.8379) (width 1.12) (layer F.Cu) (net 6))
 (segment (start 160.154091 115.840091) (end 147.141909 115.840091) (width 1.12) (layer F.Cu) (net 8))
 (segment (start 160.503 116.189) (end 160.154091 115.840091) (width 1.12) (layer F.Cu) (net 8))
 (segment (start 162.663 116.189) (end 160.503 116.189) (width 1.12) (layer F.Cu) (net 8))
 (segment (start 147.141909 115.840091) (end 146.777 116.205) (width 1.12) (layer F.Cu) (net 8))
 (segment (start 146.177 116.205) (end 146.777 116.205) (width 1.12) (layer F.Cu) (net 8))
 (segment (start 146.777 116.205) (end 147.144101 115.837899) (width 1.12) (layer F.Cu) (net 8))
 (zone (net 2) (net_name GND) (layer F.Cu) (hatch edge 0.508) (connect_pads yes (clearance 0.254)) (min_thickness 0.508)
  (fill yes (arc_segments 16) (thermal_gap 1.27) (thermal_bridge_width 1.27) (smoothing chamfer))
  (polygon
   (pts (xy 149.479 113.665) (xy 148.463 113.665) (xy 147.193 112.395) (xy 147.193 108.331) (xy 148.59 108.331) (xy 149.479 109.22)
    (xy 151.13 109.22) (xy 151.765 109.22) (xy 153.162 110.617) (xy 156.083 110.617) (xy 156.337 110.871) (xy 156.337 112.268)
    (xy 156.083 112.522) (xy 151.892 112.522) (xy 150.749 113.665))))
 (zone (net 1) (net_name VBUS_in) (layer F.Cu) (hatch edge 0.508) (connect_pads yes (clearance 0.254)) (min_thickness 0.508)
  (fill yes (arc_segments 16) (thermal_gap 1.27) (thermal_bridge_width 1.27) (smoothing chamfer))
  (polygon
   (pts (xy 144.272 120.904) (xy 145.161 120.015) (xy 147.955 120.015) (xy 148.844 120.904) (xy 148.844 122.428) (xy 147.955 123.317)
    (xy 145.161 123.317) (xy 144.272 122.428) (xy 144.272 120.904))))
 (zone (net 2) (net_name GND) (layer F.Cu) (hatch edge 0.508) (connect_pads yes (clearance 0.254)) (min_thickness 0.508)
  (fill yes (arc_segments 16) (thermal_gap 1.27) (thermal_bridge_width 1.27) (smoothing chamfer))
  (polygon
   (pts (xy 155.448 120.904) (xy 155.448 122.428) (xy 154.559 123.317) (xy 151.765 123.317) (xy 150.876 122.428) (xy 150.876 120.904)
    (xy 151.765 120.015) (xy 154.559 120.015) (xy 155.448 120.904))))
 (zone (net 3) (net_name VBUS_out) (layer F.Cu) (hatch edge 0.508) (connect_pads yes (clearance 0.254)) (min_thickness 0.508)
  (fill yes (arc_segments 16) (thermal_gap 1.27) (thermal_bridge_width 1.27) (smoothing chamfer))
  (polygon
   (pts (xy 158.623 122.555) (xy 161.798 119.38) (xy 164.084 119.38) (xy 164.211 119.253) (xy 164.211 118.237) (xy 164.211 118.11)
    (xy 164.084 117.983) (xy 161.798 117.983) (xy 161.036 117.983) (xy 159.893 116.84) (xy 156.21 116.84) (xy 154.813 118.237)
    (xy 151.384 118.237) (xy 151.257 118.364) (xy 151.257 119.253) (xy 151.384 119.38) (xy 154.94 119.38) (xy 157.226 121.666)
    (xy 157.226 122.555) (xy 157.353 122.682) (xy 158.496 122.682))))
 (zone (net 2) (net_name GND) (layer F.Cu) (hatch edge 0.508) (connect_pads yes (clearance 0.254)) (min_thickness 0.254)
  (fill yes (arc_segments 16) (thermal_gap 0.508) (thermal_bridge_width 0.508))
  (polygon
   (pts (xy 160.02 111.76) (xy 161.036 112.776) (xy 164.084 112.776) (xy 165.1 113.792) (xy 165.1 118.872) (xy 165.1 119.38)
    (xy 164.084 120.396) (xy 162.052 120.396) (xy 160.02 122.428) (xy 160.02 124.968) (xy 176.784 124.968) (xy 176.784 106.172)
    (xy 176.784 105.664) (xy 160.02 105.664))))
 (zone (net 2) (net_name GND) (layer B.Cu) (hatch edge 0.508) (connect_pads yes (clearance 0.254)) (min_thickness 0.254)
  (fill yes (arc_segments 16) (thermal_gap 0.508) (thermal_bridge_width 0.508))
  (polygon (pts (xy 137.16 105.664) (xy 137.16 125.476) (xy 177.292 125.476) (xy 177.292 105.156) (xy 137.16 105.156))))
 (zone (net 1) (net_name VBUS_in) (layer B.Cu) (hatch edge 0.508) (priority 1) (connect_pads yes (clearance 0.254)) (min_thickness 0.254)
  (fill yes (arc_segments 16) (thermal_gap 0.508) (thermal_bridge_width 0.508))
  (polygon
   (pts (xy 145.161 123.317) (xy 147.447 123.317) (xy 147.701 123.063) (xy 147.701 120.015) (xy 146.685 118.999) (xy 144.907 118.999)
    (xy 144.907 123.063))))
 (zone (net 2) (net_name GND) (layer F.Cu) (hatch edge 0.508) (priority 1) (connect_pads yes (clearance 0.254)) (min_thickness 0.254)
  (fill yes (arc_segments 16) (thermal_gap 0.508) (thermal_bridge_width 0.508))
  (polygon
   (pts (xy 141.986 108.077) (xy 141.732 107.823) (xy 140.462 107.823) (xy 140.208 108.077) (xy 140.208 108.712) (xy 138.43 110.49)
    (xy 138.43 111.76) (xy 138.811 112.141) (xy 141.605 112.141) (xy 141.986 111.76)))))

